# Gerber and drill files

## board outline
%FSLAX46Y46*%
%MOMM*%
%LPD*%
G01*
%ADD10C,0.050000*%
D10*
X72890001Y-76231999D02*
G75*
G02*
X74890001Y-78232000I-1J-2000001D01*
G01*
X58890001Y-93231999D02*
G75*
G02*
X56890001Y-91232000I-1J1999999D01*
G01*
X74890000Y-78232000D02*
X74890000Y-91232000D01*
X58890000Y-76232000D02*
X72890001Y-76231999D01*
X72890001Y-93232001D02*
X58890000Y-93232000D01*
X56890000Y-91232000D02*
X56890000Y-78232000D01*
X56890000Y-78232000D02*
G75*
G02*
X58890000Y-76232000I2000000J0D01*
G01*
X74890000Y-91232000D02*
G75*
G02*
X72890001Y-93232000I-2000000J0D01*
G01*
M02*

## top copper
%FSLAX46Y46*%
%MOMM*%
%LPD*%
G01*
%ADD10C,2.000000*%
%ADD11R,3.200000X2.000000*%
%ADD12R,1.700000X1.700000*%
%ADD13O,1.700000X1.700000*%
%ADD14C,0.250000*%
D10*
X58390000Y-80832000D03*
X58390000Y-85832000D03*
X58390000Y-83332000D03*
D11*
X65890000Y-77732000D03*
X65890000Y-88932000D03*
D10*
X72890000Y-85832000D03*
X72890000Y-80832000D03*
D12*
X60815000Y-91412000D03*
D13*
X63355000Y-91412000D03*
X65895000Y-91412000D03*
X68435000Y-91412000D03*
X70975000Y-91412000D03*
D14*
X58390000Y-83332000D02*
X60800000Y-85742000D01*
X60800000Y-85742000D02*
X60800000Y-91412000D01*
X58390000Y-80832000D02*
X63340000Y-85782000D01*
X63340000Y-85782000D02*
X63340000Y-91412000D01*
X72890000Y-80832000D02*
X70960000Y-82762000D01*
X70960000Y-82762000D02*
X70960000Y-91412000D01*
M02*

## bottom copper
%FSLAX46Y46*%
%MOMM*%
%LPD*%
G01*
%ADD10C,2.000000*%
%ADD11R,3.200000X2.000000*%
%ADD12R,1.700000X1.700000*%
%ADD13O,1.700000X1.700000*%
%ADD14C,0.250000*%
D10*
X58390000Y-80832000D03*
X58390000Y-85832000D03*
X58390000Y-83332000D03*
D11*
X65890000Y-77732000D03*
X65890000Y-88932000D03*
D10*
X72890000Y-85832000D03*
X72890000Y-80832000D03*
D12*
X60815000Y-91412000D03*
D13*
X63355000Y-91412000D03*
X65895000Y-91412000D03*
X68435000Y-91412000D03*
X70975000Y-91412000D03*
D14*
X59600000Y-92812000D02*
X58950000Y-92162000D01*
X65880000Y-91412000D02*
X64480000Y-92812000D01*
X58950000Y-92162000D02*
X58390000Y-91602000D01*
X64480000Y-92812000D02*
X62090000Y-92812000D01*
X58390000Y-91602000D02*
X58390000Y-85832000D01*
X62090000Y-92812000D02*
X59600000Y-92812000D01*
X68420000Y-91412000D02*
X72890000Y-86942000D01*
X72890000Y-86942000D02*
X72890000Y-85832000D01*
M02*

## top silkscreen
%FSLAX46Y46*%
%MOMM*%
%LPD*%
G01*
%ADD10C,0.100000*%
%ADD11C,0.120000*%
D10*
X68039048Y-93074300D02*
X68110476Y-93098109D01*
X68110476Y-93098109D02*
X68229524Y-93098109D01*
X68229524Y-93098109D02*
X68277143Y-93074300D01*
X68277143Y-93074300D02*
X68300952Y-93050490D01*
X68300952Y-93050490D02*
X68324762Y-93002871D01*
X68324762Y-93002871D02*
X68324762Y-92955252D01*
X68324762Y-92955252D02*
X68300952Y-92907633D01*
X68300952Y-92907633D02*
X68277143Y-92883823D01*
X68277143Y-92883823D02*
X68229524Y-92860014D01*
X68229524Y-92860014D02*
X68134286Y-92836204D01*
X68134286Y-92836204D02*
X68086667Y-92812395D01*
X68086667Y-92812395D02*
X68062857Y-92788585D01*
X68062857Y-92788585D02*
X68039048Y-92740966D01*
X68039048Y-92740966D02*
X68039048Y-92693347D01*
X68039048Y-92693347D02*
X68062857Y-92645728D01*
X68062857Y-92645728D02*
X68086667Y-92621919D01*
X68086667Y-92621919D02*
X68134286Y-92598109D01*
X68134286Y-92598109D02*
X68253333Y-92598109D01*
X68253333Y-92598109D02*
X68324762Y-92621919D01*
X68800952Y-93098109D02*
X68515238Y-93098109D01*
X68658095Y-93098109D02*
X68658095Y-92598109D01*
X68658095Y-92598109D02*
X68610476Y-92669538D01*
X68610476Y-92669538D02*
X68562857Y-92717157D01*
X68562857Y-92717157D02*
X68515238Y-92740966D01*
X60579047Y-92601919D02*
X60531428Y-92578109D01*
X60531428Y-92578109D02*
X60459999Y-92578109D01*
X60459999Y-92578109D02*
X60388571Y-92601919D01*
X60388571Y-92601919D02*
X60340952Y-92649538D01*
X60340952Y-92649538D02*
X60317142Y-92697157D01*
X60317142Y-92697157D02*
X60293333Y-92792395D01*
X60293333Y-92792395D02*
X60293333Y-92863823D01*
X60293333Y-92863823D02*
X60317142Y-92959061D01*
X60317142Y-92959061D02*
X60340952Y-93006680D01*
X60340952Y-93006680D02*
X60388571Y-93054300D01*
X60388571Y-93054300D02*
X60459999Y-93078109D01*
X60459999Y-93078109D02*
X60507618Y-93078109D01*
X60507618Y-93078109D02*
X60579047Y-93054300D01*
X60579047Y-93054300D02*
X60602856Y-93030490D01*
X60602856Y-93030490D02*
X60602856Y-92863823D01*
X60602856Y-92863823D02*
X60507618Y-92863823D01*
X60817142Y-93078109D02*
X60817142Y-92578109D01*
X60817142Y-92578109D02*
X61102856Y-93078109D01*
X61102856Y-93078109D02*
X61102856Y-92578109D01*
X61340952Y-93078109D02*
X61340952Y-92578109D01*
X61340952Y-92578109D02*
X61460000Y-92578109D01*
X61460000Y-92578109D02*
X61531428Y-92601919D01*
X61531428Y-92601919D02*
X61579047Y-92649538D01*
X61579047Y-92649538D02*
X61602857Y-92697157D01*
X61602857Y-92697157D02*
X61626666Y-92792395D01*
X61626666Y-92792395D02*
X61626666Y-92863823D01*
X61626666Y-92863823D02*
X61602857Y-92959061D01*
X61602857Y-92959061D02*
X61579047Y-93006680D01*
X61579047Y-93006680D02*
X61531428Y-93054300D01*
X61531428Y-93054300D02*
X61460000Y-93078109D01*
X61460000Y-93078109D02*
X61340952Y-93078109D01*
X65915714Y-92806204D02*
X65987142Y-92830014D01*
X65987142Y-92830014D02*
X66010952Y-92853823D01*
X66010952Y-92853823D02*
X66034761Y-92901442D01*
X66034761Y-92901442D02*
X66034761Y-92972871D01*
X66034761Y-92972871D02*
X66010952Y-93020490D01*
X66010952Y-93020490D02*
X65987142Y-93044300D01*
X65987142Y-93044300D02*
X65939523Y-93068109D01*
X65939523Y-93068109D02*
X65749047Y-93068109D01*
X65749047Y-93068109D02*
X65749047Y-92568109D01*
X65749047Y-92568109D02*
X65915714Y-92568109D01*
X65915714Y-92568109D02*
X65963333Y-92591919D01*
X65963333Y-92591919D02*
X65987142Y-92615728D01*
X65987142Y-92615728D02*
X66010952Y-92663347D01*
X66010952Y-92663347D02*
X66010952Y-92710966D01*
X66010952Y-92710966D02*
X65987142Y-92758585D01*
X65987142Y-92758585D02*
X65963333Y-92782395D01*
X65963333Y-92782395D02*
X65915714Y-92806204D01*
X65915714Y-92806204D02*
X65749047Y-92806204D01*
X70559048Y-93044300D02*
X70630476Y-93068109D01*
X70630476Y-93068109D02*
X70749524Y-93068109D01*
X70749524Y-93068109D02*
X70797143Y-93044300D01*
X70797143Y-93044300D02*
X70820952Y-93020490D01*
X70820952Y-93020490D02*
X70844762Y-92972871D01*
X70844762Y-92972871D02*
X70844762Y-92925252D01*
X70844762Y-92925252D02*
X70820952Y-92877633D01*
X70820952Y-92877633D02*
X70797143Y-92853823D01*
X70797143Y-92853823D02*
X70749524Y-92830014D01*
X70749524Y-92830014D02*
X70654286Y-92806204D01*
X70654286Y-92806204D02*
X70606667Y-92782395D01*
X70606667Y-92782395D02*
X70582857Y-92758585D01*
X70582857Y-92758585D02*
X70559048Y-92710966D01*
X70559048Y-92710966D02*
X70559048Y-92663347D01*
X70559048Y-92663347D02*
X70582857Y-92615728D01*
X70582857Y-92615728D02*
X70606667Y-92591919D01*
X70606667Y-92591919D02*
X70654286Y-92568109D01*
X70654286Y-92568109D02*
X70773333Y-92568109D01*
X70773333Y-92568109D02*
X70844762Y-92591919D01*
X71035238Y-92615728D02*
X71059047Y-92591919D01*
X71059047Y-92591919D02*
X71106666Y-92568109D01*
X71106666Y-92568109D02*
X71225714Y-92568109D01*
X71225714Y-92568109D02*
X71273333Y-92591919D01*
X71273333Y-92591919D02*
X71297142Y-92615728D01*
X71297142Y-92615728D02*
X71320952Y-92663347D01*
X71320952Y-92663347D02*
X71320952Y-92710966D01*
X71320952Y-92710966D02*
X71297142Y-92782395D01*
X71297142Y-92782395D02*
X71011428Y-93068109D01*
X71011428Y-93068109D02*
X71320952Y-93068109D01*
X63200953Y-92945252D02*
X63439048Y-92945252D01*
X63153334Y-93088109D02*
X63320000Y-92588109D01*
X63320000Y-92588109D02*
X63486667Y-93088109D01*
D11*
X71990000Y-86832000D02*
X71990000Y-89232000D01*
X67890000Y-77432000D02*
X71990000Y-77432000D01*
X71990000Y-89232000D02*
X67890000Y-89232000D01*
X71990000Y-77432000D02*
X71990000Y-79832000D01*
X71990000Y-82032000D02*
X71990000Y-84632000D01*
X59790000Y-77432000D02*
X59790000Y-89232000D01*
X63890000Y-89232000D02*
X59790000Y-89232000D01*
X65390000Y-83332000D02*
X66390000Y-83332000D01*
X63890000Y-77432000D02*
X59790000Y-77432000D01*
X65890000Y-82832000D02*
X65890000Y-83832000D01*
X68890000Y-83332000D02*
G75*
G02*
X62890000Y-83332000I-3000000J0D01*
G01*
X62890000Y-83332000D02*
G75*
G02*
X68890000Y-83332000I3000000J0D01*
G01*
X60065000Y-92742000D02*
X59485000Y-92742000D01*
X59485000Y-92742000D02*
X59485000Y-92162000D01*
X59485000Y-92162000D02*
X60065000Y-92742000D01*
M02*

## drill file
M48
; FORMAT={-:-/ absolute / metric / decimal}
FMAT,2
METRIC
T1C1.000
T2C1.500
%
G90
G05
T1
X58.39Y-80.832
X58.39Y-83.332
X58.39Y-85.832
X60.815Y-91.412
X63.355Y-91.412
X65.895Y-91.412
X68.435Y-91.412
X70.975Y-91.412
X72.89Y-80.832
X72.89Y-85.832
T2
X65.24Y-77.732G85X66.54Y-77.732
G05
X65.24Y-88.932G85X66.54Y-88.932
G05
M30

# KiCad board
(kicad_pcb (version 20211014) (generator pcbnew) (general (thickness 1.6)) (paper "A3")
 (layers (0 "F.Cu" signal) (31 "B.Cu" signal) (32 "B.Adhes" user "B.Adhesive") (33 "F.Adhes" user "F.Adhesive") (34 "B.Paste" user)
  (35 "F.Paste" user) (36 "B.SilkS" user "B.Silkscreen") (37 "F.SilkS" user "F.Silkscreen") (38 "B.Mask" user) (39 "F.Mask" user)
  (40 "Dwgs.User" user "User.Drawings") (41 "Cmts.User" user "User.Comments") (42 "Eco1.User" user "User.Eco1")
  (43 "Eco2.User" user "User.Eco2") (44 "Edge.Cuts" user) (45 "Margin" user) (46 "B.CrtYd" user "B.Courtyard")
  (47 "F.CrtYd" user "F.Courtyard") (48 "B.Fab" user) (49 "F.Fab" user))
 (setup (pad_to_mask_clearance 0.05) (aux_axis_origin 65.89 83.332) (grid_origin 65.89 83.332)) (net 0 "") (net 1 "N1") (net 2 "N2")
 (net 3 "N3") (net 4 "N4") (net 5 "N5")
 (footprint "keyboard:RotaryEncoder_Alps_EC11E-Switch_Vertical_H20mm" (layer "F.Cu") (at 65.89 83.332)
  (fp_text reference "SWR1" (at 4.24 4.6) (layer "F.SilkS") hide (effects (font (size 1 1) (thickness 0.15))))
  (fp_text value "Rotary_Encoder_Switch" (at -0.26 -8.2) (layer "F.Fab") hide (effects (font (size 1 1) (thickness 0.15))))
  (fp_line (start 6.1 3.5) (end 6.1 5.9) (layer "F.SilkS") (width 0.12))
  (fp_line (start 2 -5.9) (end 6.1 -5.9) (layer "F.SilkS") (width 0.12))
  (fp_line (start 6.1 5.9) (end 2 5.9) (layer "F.SilkS") (width 0.12))
  (fp_line (start 6.1 -5.9) (end 6.1 -3.5) (layer "F.SilkS") (width 0.12))
  (fp_line (start 6.1 -1.3) (end 6.1 1.3) (layer "F.SilkS") (width 0.12))
  (fp_line (start -6.1 -5.9) (end -6.1 5.9) (layer "F.SilkS") (width 0.12))
  (fp_line (start -2 5.9) (end -6.1 5.9) (layer "F.SilkS") (width 0.12))
  (fp_line (start -0.5 0) (end 0.5 0) (layer "F.SilkS") (width 0.12))
  (fp_line (start -2 -5.9) (end -6.1 -5.9) (layer "F.SilkS") (width 0.12))
  (fp_line (start 0 -0.5) (end 0 0.5) (layer "F.SilkS") (width 0.12))
  (fp_circle (center 0 0) (end 3 0) (layer "F.SilkS") (width 0.12) (fill none))
  (pad "A" thru_hole circle (at -7.5 -2.5) (size 2 2) (drill 1) (layers *.Cu *.Mask) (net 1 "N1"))
  (pad "B" thru_hole circle (at -7.5 2.5) (size 2 2) (drill 1) (layers *.Cu *.Mask) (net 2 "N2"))
  (pad "C" thru_hole circle (at -7.5 0) (size 2 2) (drill 1) (layers *.Cu *.Mask) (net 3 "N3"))
  (pad "MP" thru_hole rect (at 0 -5.6) (size 3.2 2) (drill oval 2.8 1.5) (layers *.Cu *.Mask))
  (pad "MP" thru_hole rect (at 0 5.6) (size 3.2 2) (drill oval 2.8 1.5) (layers *.Cu *.Mask))
  (pad "S1" thru_hole circle (at 7 2.5) (size 2 2) (drill 1) (layers *.Cu *.Mask) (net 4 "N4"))
  (pad "S2" thru_hole circle (at 7 -2.5) (size 2 2) (drill 1) (layers *.Cu *.Mask) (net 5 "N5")))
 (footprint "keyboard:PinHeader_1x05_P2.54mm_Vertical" (layer "F.Cu") (at 60.815 91.412 90)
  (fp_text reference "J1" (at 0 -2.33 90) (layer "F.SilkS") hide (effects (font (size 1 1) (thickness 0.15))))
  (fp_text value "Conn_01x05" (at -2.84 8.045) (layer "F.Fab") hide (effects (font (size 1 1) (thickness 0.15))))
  (fp_line (start -1.33 -0.75) (end -1.33 -1.33) (layer "F.SilkS") (width 0.12))
  (fp_line (start -1.33 -1.33) (end -0.75 -1.33) (layer "F.SilkS") (width 0.12))
  (fp_line (start -0.75 -1.33) (end -1.33 -0.75) (layer "F.SilkS") (width 0.12))
  (pad "1" thru_hole rect (at 0 0 90) (size 1.7 1.7) (drill 1) (layers *.Cu *.Mask) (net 3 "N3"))
  (pad "2" thru_hole oval (at 0 2.54 90) (size 1.7 1.7) (drill 1) (layers *.Cu *.Mask) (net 1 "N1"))
  (pad "3" thru_hole oval (at 0 5.08 90) (size 1.7 1.7) (drill 1) (layers *.Cu *.Mask) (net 2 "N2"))
  (pad "4" thru_hole oval (at 0 7.62 90) (size 1.7 1.7) (drill 1) (layers *.Cu *.Mask) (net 4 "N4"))
  (pad "5" thru_hole oval (at 0 10.16 90) (size 1.7 1.7) (drill 1) (layers *.Cu *.Mask) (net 5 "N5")))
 (gr_arc (start 72.890001 76.231999) (mid 74.304215 76.817785) (end 74.89 78.232) (layer "Edge.Cuts") (width 0.05))
 (gr_arc (start 58.890001 93.231999) (mid 57.475787 92.646214) (end 56.89 91.232) (layer "Edge.Cuts") (width 0.05))
 (gr_line (start 74.89 78.232) (end 74.89 91.232) (layer "Edge.Cuts") (width 0.05))
 (gr_line (start 58.89 76.232) (end 72.890001 76.231999) (layer "Edge.Cuts") (width 0.05))
 (gr_line (start 72.890001 93.232001) (end 58.89 93.232) (layer "Edge.Cuts") (width 0.05))
 (gr_line (start 56.89 91.232) (end 56.89 78.232) (layer "Edge.Cuts") (width 0.05))
 (gr_arc (start 56.89 78.232) (mid 57.475786 76.817786) (end 58.89 76.232) (layer "Edge.Cuts") (width 0.05))
 (gr_arc (start 74.89 91.232) (mid 74.304215 92.646214) (end 72.890001 93.232001) (layer "Edge.Cuts") (width 0.05))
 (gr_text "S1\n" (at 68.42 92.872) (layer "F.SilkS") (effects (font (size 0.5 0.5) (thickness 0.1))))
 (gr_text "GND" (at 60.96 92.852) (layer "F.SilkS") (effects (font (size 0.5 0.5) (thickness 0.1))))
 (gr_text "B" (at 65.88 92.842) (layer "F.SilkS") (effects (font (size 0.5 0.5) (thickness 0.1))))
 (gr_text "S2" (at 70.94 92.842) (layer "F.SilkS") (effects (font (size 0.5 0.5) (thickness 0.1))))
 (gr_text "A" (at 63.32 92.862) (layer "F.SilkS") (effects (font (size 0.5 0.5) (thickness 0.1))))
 (segment (start 58.39 83.332) (end 60.8 85.742) (width 0.25) (layer "F.Cu") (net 3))
 (segment (start 60.8 85.742) (end 60.8 91.412) (width 0.25) (layer "F.Cu") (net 3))
 (segment (start 58.39 80.832) (end 63.34 85.782) (width 0.25) (layer "F.Cu") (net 1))
 (segment (start 63.34 85.782) (end 63.34 91.412) (width 0.25) (layer "F.Cu") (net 1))
 (segment (start 59.6 92.812) (end 58.95 92.162) (width 0.25) (layer "B.Cu") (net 2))
 (segment (start 65.88 91.412) (end 64.48 92.812) (width 0.25) (layer "B.Cu") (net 2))
 (segment (start 58.95 92.162) (end 58.39 91.602) (width 0.25) (layer "B.Cu") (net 2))
 (segment (start 64.48 92.812) (end 62.09 92.812) (width 0.25) (layer "B.Cu") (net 2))
 (segment (start 58.39 91.602) (end 58.39 85.832) (width 0.25) (layer "B.Cu") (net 2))
 (segment (start 62.09 92.812) (end 59.6 92.812) (width 0.25) (layer "B.Cu") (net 2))
 (segment (start 68.42 91.412) (end 72.89 86.942) (width 0.25) (layer "B.Cu") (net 4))
 (segment (start 72.89 86.942) (end 72.89 85.832) (width 0.25) (layer "B.Cu") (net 4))
 (segment (start 72.89 80.832) (end 70.96 82.762) (width 0.25) (layer "F.Cu") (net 5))
 (segment (start 70.96 82.762) (end 70.96 91.412) (width 0.25) (layer "F.Cu") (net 5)))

